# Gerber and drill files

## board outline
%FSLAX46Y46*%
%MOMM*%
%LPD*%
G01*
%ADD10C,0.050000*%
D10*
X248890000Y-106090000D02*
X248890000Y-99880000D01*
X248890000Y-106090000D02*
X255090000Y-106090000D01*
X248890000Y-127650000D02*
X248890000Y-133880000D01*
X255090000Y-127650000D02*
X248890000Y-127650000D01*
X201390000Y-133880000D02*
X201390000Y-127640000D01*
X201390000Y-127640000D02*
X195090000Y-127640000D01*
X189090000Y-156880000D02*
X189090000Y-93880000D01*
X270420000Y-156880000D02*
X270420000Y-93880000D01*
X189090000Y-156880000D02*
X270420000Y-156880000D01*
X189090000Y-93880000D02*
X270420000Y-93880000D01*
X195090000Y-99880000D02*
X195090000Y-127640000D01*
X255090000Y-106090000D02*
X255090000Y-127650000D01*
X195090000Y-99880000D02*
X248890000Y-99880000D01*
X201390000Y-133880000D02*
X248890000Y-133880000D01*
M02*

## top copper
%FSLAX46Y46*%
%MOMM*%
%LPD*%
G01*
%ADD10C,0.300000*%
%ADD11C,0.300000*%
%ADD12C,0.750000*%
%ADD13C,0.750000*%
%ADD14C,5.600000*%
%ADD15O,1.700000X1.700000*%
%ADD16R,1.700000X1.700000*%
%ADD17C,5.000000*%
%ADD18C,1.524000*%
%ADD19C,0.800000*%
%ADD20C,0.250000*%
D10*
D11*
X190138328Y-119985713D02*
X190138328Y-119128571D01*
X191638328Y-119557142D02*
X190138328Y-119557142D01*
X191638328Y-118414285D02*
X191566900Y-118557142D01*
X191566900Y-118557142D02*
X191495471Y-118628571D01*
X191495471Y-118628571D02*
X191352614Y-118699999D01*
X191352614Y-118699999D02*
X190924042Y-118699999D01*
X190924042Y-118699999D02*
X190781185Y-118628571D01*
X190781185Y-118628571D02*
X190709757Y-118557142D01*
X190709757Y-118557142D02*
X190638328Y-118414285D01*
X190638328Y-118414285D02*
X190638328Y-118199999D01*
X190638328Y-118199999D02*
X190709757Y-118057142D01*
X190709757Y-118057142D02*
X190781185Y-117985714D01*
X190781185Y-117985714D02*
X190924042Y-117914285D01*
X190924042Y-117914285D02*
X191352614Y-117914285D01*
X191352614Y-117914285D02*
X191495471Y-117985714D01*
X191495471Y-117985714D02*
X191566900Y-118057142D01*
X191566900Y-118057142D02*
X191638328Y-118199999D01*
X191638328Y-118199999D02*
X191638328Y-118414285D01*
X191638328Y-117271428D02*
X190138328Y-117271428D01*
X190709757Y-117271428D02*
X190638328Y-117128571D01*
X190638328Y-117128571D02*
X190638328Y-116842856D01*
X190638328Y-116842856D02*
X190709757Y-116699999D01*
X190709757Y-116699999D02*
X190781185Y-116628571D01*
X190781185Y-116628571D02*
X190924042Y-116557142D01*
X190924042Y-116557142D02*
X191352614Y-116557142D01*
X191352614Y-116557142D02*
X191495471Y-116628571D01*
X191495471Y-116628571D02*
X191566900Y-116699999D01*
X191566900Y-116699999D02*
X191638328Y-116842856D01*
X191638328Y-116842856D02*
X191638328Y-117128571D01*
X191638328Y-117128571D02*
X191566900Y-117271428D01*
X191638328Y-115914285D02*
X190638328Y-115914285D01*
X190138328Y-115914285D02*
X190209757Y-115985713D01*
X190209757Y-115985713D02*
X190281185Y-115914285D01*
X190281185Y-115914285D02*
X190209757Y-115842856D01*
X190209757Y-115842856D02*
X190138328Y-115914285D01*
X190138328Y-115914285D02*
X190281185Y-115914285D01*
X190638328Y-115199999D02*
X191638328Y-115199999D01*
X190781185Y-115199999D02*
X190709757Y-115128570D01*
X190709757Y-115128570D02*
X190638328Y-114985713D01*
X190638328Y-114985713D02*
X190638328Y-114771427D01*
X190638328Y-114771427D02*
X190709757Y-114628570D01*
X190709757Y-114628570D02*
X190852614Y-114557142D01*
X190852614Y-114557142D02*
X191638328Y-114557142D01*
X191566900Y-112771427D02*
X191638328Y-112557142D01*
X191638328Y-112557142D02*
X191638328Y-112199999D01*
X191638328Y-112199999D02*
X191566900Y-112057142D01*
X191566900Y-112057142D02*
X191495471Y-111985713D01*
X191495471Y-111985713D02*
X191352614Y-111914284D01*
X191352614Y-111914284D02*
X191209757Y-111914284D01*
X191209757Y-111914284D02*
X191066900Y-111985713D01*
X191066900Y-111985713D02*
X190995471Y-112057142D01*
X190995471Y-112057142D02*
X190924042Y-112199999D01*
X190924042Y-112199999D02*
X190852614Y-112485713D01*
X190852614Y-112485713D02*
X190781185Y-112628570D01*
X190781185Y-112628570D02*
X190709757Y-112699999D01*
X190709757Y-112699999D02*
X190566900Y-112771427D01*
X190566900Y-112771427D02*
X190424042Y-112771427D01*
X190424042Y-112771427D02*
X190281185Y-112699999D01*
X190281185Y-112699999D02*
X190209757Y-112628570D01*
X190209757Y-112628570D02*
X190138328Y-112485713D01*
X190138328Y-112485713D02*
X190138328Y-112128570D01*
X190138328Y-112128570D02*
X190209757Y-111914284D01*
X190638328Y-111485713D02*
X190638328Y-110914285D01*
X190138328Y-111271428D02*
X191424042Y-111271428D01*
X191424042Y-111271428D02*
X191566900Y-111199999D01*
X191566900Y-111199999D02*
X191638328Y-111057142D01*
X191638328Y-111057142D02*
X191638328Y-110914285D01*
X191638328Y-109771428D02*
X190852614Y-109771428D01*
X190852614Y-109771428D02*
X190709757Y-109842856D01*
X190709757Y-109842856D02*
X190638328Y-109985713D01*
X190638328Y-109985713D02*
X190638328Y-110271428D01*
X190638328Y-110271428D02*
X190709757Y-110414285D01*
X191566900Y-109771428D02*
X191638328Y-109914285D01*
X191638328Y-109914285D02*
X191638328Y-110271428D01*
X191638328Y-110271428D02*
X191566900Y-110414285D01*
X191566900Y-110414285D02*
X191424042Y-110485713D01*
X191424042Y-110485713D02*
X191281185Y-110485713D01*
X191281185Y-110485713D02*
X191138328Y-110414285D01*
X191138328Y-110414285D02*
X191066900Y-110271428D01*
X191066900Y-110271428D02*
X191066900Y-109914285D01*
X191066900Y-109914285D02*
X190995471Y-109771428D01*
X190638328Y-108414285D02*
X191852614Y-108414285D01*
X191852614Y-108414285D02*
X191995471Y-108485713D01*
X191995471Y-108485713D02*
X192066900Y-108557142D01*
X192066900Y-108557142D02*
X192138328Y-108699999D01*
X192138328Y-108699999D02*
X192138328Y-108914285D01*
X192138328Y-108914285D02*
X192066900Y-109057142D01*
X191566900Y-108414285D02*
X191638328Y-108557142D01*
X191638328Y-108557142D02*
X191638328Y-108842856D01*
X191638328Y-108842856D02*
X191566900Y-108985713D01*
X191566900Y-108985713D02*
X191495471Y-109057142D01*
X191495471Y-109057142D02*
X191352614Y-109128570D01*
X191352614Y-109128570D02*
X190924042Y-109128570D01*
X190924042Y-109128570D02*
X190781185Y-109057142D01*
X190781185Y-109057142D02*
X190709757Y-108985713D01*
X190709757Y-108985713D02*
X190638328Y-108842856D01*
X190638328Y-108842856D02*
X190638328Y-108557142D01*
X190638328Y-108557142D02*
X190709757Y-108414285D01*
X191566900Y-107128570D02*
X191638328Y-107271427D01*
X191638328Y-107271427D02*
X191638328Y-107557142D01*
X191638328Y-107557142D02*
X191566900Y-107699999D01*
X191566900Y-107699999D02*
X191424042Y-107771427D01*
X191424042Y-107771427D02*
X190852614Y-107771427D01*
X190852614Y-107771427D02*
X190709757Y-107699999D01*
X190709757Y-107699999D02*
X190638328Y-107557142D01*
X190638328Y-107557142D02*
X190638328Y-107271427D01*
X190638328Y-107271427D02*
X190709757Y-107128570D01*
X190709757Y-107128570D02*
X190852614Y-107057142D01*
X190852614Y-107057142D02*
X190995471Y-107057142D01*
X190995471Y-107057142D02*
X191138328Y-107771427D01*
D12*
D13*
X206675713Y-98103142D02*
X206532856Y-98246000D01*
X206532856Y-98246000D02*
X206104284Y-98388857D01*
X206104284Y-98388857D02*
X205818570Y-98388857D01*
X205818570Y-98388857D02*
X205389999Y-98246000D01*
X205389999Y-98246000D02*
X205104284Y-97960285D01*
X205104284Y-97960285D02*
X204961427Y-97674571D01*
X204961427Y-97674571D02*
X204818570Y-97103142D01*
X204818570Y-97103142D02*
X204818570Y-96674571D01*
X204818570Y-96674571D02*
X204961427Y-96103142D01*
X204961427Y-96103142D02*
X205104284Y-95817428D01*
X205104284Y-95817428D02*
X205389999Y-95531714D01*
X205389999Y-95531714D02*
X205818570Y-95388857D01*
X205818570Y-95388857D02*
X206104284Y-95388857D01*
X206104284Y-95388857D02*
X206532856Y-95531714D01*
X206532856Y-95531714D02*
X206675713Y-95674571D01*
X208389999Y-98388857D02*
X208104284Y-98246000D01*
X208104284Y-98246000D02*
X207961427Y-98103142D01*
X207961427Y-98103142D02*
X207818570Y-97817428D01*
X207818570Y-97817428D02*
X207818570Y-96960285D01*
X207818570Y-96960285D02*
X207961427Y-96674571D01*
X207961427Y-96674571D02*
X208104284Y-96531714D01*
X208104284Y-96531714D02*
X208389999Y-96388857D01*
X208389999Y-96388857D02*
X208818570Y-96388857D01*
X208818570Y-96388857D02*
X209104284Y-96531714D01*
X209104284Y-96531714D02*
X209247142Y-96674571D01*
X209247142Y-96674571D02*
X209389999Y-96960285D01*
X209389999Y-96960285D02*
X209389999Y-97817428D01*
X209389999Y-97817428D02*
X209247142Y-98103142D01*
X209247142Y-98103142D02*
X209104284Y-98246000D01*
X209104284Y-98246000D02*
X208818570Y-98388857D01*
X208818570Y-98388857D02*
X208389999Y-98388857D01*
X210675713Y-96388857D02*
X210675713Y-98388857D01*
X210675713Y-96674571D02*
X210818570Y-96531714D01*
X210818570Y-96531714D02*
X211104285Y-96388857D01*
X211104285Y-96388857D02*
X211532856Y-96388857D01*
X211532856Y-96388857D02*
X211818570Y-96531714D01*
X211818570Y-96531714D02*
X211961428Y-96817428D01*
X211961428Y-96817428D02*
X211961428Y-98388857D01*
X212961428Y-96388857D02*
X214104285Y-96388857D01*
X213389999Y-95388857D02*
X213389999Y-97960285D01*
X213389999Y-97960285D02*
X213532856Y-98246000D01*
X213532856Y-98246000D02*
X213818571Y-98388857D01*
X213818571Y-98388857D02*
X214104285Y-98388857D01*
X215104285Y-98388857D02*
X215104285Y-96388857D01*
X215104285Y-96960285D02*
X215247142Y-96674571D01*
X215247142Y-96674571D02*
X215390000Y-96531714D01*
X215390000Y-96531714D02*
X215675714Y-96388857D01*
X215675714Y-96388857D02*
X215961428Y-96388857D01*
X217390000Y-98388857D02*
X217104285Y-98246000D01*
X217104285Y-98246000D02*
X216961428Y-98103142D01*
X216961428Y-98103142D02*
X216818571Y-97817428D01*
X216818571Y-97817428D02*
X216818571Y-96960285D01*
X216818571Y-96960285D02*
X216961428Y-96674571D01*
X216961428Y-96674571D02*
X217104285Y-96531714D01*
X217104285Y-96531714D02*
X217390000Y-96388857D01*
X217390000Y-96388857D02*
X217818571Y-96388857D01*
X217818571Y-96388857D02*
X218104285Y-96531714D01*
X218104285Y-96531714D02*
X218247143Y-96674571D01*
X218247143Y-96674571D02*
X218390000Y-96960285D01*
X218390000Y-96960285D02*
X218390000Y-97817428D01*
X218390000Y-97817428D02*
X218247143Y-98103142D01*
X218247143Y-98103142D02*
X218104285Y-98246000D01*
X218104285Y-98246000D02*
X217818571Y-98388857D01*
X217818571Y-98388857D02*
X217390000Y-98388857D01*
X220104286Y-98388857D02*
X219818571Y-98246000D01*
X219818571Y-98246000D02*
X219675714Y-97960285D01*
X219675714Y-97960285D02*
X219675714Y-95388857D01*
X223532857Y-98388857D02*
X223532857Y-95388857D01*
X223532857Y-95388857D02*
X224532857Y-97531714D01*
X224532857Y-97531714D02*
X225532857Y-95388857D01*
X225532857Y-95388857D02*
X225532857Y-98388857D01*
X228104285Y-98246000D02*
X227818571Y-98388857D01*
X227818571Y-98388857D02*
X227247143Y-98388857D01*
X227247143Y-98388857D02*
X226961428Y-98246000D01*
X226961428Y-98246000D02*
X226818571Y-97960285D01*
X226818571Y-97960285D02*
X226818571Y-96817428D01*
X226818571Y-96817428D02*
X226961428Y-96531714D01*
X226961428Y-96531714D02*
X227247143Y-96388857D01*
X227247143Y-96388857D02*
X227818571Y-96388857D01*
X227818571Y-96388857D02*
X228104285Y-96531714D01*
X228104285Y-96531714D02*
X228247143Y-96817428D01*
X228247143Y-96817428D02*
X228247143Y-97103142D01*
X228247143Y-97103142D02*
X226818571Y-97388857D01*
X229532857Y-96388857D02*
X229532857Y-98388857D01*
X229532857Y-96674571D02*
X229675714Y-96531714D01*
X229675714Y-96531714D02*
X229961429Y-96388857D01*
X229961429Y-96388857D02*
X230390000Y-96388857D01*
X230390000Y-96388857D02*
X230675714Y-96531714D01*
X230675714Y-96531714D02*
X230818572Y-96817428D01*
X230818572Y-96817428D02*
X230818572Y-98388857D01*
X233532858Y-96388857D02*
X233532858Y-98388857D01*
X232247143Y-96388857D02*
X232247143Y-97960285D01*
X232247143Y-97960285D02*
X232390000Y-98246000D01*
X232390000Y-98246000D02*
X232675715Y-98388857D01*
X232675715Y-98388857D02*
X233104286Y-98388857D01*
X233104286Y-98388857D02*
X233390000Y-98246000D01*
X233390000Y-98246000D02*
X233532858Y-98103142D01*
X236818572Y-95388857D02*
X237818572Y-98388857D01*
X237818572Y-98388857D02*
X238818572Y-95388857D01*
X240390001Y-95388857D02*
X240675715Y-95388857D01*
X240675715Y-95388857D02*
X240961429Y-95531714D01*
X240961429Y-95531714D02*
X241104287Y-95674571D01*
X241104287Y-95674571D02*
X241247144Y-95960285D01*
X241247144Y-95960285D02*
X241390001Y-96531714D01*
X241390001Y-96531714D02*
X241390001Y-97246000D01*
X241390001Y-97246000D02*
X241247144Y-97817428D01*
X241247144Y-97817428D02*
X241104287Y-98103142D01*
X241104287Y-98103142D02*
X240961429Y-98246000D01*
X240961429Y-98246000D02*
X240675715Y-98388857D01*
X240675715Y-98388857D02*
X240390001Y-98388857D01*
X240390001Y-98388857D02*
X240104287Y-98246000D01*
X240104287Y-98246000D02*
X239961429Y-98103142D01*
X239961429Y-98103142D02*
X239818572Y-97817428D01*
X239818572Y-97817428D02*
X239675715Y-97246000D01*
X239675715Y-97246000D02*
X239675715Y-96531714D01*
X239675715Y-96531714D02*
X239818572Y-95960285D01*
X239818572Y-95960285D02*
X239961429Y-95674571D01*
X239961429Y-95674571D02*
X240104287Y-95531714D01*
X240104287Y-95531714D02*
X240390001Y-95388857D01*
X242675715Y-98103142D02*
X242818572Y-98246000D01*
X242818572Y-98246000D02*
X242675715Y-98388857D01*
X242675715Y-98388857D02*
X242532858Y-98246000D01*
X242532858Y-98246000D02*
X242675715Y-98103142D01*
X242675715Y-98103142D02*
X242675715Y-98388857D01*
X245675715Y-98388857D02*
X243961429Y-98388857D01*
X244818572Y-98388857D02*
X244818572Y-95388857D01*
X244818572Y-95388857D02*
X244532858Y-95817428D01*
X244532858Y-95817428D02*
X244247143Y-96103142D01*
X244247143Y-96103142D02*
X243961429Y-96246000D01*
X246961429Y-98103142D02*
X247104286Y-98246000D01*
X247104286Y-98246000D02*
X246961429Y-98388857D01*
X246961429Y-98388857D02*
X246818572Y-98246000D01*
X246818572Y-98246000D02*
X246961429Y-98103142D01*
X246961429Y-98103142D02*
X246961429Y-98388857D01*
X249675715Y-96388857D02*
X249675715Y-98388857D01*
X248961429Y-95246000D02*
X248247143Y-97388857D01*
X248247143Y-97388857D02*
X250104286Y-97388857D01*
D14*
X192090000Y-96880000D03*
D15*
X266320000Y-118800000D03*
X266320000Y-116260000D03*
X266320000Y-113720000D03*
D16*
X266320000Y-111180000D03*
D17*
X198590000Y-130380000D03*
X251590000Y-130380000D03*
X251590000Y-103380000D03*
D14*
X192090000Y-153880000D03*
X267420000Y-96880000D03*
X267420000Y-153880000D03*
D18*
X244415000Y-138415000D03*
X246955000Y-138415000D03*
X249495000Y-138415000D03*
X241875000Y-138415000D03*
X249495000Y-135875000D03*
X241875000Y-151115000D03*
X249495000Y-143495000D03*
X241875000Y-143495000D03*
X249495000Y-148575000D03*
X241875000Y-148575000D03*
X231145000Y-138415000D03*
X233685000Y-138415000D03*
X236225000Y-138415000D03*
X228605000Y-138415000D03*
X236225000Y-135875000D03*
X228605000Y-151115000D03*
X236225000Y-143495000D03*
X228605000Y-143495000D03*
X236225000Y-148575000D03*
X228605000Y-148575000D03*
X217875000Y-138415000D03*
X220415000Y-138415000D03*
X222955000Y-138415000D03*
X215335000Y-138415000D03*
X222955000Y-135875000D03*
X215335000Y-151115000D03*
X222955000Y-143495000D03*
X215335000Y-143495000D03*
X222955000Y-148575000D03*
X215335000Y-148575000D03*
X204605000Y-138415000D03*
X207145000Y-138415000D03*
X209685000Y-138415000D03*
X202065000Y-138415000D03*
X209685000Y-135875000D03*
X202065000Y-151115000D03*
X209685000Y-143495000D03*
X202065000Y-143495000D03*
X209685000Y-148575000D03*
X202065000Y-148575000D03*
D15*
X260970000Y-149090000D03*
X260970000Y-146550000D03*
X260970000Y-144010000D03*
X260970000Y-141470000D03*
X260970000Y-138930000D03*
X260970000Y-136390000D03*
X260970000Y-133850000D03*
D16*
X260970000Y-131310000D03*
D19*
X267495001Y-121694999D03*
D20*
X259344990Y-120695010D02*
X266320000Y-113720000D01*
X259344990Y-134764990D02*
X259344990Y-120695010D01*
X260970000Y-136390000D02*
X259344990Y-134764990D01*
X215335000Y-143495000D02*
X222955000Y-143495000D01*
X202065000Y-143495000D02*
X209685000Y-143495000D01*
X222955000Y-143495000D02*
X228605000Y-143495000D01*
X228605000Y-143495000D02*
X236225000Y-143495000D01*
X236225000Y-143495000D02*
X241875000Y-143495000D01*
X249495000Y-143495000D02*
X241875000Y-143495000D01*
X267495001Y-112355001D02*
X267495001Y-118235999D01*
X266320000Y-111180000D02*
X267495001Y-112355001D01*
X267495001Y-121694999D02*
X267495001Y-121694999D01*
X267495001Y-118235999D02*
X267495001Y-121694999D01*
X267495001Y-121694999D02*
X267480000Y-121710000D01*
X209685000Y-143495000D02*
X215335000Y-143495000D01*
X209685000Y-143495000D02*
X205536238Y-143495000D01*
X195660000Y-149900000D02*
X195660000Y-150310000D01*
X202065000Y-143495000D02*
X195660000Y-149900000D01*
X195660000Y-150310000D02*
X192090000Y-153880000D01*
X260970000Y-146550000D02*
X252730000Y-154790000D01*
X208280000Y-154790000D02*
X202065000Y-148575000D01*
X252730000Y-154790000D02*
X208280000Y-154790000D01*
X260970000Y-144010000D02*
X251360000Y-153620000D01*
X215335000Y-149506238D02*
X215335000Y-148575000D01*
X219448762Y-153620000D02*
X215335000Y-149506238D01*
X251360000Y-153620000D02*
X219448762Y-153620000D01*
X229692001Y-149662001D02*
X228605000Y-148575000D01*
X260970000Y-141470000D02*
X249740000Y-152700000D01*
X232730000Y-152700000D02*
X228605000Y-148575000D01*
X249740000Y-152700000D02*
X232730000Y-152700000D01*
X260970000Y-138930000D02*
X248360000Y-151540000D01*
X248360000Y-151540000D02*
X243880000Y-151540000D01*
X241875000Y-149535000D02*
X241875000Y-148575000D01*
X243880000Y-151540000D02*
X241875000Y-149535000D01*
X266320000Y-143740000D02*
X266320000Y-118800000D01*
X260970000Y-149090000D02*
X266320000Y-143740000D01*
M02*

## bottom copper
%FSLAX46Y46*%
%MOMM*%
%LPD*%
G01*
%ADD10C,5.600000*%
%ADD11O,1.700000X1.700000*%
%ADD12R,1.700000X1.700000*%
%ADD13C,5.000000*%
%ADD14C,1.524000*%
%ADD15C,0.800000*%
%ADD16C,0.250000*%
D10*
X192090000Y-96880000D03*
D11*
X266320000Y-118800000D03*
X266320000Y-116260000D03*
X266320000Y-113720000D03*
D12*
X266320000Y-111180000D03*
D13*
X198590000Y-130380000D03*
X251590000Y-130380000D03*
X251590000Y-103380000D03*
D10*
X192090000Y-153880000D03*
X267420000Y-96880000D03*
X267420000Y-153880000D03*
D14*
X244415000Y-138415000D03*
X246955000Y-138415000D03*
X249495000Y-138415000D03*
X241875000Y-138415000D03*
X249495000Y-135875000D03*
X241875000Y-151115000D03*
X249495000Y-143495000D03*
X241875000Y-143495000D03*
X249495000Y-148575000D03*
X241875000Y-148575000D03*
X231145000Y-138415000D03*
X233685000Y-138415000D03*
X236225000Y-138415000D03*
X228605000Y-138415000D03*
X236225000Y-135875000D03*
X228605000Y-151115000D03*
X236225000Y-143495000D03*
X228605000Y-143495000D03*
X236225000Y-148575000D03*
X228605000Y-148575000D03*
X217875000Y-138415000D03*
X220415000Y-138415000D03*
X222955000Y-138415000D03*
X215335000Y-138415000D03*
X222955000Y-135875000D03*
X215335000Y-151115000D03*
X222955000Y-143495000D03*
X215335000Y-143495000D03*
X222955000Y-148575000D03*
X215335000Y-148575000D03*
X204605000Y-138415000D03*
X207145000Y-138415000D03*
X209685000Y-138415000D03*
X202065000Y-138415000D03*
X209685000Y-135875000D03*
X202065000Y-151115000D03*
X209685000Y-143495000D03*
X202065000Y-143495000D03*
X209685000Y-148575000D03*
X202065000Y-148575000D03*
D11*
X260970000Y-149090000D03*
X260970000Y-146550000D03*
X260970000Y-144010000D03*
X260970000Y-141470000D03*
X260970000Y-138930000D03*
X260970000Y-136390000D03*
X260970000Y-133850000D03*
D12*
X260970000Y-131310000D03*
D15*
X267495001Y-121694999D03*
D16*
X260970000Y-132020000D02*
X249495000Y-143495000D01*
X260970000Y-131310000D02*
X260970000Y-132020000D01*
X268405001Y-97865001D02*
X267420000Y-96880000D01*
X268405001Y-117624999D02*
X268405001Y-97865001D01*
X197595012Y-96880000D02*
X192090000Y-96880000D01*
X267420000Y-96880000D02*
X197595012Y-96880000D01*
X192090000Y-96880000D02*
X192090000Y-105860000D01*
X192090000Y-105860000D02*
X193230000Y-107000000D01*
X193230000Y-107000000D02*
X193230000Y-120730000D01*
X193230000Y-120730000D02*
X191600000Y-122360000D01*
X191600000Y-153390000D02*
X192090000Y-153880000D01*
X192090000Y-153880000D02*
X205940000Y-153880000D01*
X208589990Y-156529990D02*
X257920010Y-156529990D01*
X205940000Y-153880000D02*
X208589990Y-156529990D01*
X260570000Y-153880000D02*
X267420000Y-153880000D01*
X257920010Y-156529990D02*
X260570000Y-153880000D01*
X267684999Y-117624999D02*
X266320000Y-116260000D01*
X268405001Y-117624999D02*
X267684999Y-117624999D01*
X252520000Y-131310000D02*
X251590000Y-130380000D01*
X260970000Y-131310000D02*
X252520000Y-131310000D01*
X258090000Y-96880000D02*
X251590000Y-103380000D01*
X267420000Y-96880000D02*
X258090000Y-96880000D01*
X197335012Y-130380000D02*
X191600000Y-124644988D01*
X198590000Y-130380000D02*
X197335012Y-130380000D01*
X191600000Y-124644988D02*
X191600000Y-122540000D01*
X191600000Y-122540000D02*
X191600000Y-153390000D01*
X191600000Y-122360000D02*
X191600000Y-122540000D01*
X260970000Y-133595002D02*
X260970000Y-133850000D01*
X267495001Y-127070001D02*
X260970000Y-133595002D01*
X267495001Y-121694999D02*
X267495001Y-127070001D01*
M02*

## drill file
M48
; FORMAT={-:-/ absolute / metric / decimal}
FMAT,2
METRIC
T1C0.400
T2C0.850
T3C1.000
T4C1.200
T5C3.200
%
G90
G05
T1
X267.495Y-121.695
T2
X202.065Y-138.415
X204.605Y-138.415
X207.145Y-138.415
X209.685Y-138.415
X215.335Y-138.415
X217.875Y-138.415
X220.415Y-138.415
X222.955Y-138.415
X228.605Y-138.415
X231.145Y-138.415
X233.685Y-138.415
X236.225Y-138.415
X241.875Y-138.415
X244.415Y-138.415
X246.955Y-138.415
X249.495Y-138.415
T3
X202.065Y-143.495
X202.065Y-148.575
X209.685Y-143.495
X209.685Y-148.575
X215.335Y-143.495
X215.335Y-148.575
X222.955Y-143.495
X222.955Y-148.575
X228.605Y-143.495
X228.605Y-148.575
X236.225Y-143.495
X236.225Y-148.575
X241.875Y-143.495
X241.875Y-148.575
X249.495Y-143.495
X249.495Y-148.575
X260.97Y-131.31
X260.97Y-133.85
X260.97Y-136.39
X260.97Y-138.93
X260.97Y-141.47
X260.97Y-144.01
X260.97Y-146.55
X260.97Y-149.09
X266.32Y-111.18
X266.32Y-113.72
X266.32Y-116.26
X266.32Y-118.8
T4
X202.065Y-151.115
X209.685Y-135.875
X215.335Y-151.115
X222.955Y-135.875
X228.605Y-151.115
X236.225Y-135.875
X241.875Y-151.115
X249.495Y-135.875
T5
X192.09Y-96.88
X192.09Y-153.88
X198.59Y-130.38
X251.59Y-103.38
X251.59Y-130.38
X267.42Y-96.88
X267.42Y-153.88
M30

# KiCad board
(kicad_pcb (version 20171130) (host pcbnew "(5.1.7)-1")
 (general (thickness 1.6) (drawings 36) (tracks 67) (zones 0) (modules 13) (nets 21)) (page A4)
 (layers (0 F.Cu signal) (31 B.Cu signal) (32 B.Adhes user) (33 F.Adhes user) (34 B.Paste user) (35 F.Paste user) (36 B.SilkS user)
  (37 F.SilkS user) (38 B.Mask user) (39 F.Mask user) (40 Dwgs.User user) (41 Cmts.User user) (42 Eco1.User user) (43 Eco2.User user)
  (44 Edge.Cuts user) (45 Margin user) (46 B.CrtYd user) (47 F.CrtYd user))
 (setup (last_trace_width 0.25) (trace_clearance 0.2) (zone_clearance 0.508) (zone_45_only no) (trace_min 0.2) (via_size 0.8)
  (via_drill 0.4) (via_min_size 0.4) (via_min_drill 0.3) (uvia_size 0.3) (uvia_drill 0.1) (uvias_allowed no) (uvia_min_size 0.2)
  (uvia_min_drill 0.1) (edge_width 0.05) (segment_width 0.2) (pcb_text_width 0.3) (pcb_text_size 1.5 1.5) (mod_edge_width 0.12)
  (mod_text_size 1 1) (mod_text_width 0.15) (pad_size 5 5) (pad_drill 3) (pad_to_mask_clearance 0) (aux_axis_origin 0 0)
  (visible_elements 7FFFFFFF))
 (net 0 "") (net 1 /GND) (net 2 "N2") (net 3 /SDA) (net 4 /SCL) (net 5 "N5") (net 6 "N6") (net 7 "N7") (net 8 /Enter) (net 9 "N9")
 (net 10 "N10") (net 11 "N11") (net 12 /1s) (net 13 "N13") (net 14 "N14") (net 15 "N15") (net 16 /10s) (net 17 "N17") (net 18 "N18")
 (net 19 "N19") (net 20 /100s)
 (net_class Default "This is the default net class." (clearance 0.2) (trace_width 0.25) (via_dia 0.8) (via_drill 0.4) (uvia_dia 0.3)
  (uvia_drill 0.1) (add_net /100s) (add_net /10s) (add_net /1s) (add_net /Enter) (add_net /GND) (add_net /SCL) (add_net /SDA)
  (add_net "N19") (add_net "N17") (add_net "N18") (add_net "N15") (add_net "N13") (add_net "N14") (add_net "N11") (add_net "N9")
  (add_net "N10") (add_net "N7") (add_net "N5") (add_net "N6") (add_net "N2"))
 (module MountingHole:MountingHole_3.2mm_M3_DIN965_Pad (layer F.Cu) (at 192.09 96.88)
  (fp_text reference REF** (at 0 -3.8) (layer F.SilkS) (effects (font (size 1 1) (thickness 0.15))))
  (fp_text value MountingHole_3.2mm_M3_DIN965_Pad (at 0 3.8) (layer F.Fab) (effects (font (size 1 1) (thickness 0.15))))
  (pad 1 thru_hole circle (at 0 0) (size 5.6 5.6) (drill 3.2) (layers *.Cu *.Mask) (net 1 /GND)))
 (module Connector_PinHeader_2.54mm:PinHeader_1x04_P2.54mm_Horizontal (layer B.Cu) (at 266.32 111.18 180)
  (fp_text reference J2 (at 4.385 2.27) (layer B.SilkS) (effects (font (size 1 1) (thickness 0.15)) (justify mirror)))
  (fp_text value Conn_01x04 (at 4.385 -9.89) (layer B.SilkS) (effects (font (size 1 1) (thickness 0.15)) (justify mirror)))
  (pad 4 thru_hole oval (at 0 -7.62 180) (size 1.7 1.7) (drill 1) (layers *.Cu *.Mask) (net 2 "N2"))
  (pad 3 thru_hole oval (at 0 -5.08 180) (size 1.7 1.7) (drill 1) (layers *.Cu *.Mask) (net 1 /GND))
  (pad 2 thru_hole oval (at 0 -2.54 180) (size 1.7 1.7) (drill 1) (layers *.Cu *.Mask) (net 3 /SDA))
  (pad 1 thru_hole rect (at 0 0 180) (size 1.7 1.7) (drill 1) (layers *.Cu *.Mask) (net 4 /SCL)))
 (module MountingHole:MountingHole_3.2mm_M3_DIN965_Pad (layer F.Cu) (at 198.59 130.38)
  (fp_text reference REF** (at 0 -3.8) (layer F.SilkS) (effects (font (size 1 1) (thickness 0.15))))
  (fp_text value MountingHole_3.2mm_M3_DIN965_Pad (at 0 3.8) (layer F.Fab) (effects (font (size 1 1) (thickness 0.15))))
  (pad 1 thru_hole circle (at 0 0) (size 5 5) (drill 3.2) (layers *.Cu *.Mask) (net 1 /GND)))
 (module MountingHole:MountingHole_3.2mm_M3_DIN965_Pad (layer F.Cu) (at 251.59 130.38)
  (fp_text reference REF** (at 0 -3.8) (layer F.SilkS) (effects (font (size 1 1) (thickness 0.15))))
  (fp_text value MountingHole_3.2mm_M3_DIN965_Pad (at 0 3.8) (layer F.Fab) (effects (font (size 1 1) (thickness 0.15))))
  (pad 1 thru_hole circle (at 0 0) (size 5 5) (drill 3.2) (layers *.Cu *.Mask) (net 1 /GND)))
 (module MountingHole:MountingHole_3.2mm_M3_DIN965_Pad (layer F.Cu) (at 251.59 103.38)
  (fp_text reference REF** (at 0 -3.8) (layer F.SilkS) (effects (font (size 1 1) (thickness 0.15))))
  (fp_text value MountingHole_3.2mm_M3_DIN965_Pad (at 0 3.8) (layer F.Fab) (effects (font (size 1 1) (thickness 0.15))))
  (pad 1 thru_hole circle (at 0 0) (size 5 5) (drill 3.2) (layers *.Cu *.Mask) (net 1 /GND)))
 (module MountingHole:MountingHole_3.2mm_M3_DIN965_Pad (layer F.Cu) (at 192.09 153.88)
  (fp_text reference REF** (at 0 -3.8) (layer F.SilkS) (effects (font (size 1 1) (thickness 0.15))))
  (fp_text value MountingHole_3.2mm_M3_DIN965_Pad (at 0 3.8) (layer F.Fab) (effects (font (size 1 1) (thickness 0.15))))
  (pad 1 thru_hole circle (at 0 0) (size 5.6 5.6) (drill 3.2) (layers *.Cu *.Mask) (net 1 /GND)))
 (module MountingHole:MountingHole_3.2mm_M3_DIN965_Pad (layer F.Cu) (at 267.42 96.88)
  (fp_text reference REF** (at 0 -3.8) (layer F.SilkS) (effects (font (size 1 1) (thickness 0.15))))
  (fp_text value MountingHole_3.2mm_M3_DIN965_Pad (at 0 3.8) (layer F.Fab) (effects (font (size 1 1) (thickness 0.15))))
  (pad 1 thru_hole circle (at 0 0) (size 5.6 5.6) (drill 3.2) (layers *.Cu *.Mask) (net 1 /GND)))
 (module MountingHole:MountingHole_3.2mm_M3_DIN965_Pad (layer F.Cu) (at 267.42 153.88)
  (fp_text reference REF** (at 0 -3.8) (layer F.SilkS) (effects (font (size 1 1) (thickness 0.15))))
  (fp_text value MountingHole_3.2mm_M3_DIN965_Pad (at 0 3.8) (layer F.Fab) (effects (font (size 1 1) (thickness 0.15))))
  (pad 1 thru_hole circle (at 0 0) (size 5.6 5.6) (drill 3.2) (layers *.Cu *.Mask) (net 1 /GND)))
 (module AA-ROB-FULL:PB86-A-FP (layer F.Cu) (at 239.515 134.995)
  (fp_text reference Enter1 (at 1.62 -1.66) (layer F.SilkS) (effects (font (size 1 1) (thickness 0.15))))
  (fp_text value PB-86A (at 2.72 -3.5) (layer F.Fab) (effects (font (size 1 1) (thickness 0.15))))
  (pad 5 thru_hole circle (at 4.9 3.42) (size 1.524 1.524) (drill 0.85) (layers *.Cu *.Mask) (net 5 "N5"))
  (pad 6 thru_hole circle (at 7.44 3.42) (size 1.524 1.524) (drill 0.85) (layers *.Cu *.Mask) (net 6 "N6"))
  (pad 7 thru_hole circle (at 9.98 3.42) (size 1.524 1.524) (drill 0.85) (layers *.Cu *.Mask))
  (pad 4 thru_hole circle (at 2.36 3.42) (size 1.524 1.524) (drill 0.85) (layers *.Cu *.Mask))
  (pad 8 thru_hole circle (at 9.98 0.88) (size 1.524 1.524) (drill 1.2) (layers *.Cu *.Mask))
  (pad 8 thru_hole circle (at 2.36 16.12) (size 1.524 1.524) (drill 1.2) (layers *.Cu *.Mask))
  (pad 1 thru_hole circle (at 9.98 8.5) (size 1.524 1.524) (drill 1) (layers *.Cu *.Mask) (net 1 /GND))
  (pad 1 thru_hole circle (at 2.36 8.5) (size 1.524 1.524) (drill 1) (layers *.Cu *.Mask) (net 1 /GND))
  (pad 3 thru_hole circle (at 9.98 13.58) (size 1.524 1.524) (drill 1) (layers *.Cu *.Mask) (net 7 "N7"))
  (pad 2 thru_hole circle (at 2.36 13.58) (size 1.524 1.524) (drill 1) (layers *.Cu *.Mask) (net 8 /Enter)))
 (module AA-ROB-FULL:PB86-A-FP (layer F.Cu) (at 226.245 134.995)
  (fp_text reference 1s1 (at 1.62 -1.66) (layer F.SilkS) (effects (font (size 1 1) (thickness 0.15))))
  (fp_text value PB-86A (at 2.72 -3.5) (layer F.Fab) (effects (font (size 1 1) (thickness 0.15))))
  (pad 5 thru_hole circle (at 4.9 3.42) (size 1.524 1.524) (drill 0.85) (layers *.Cu *.Mask) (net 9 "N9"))
  (pad 6 thru_hole circle (at 7.44 3.42) (size 1.524 1.524) (drill 0.85) (layers *.Cu *.Mask) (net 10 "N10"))
  (pad 7 thru_hole circle (at 9.98 3.42) (size 1.524 1.524) (drill 0.85) (layers *.Cu *.Mask))
  (pad 4 thru_hole circle (at 2.36 3.42) (size 1.524 1.524) (drill 0.85) (layers *.Cu *.Mask))
  (pad 8 thru_hole circle (at 9.98 0.88) (size 1.524 1.524) (drill 1.2) (layers *.Cu *.Mask))
  (pad 8 thru_hole circle (at 2.36 16.12) (size 1.524 1.524) (drill 1.2) (layers *.Cu *.Mask))
  (pad 1 thru_hole circle (at 9.98 8.5) (size 1.524 1.524) (drill 1) (layers *.Cu *.Mask) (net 1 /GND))
  (pad 1 thru_hole circle (at 2.36 8.5) (size 1.524 1.524) (drill 1) (layers *.Cu *.Mask) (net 1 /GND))
  (pad 3 thru_hole circle (at 9.98 13.58) (size 1.524 1.524) (drill 1) (layers *.Cu *.Mask) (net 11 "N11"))
  (pad 2 thru_hole circle (at 2.36 13.58) (size 1.524 1.524) (drill 1) (layers *.Cu *.Mask) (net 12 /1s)))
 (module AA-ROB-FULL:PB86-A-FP (layer F.Cu) (at 212.975 134.995)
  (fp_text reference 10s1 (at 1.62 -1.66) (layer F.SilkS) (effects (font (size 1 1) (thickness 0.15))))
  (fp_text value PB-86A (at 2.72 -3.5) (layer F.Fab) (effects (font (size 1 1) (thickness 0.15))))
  (pad 5 thru_hole circle (at 4.9 3.42) (size 1.524 1.524) (drill 0.85) (layers *.Cu *.Mask) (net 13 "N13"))
  (pad 6 thru_hole circle (at 7.44 3.42) (size 1.524 1.524) (drill 0.85) (layers *.Cu *.Mask) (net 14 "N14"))
  (pad 7 thru_hole circle (at 9.98 3.42) (size 1.524 1.524) (drill 0.85) (layers *.Cu *.Mask))
  (pad 4 thru_hole circle (at 2.36 3.42) (size 1.524 1.524) (drill 0.85) (layers *.Cu *.Mask))
  (pad 8 thru_hole circle (at 9.98 0.88) (size 1.524 1.524) (drill 1.2) (layers *.Cu *.Mask))
  (pad 8 thru_hole circle (at 2.36 16.12) (size 1.524 1.524) (drill 1.2) (layers *.Cu *.Mask))
  (pad 1 thru_hole circle (at 9.98 8.5) (size 1.524 1.524) (drill 1) (layers *.Cu *.Mask) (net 1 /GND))
  (pad 1 thru_hole circle (at 2.36 8.5) (size 1.524 1.524) (drill 1) (layers *.Cu *.Mask) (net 1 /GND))
  (pad 3 thru_hole circle (at 9.98 13.58) (size 1.524 1.524) (drill 1) (layers *.Cu *.Mask) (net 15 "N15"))
  (pad 2 thru_hole circle (at 2.36 13.58) (size 1.524 1.524) (drill 1) (layers *.Cu *.Mask) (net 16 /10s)))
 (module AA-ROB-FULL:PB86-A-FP (layer F.Cu) (at 199.705 134.995)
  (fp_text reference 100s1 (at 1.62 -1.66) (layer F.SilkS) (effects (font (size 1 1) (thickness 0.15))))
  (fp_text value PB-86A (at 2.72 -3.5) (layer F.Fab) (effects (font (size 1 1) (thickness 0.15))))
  (pad 5 thru_hole circle (at 4.9 3.42) (size 1.524 1.524) (drill 0.85) (layers *.Cu *.Mask) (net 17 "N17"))
  (pad 6 thru_hole circle (at 7.44 3.42) (size 1.524 1.524) (drill 0.85) (layers *.Cu *.Mask) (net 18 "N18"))
  (pad 7 thru_hole circle (at 9.98 3.42) (size 1.524 1.524) (drill 0.85) (layers *.Cu *.Mask))
  (pad 4 thru_hole circle (at 2.36 3.42) (size 1.524 1.524) (drill 0.85) (layers *.Cu *.Mask))
  (pad 8 thru_hole circle (at 9.98 0.88) (size 1.524 1.524) (drill 1.2) (layers *.Cu *.Mask))
  (pad 8 thru_hole circle (at 2.36 16.12) (size 1.524 1.524) (drill 1.2) (layers *.Cu *.Mask))
  (pad 1 thru_hole circle (at 9.98 8.5) (size 1.524 1.524) (drill 1) (layers *.Cu *.Mask) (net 1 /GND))
  (pad 1 thru_hole circle (at 2.36 8.5) (size 1.524 1.524) (drill 1) (layers *.Cu *.Mask) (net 1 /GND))
  (pad 3 thru_hole circle (at 9.98 13.58) (size 1.524 1.524) (drill 1) (layers *.Cu *.Mask) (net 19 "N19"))
  (pad 2 thru_hole circle (at 2.36 13.58) (size 1.524 1.524) (drill 1) (layers *.Cu *.Mask) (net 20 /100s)))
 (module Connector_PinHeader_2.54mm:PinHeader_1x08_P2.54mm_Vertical (layer F.Cu) (at 260.97 131.31)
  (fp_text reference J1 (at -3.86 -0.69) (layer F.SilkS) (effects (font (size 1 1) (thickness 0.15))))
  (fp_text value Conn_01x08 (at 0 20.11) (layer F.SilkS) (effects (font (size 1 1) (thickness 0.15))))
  (pad 8 thru_hole oval (at 0 17.78) (size 1.7 1.7) (drill 1) (layers *.Cu *.Mask) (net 2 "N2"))
  (pad 7 thru_hole oval (at 0 15.24) (size 1.7 1.7) (drill 1) (layers *.Cu *.Mask) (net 20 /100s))
  (pad 6 thru_hole oval (at 0 12.7) (size 1.7 1.7) (drill 1) (layers *.Cu *.Mask) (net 16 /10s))
  (pad 5 thru_hole oval (at 0 10.16) (size 1.7 1.7) (drill 1) (layers *.Cu *.Mask) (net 12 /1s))
  (pad 4 thru_hole oval (at 0 7.62) (size 1.7 1.7) (drill 1) (layers *.Cu *.Mask) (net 8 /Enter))
  (pad 3 thru_hole oval (at 0 5.08) (size 1.7 1.7) (drill 1) (layers *.Cu *.Mask) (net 3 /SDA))
  (pad 2 thru_hole oval (at 0 2.54) (size 1.7 1.7) (drill 1) (layers *.Cu *.Mask) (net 4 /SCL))
  (pad 1 thru_hole rect (at 0 0) (size 1.7 1.7) (drill 1) (layers *.Cu *.Mask) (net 1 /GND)))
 (gr_line (start 248.89 106.09) (end 248.89 99.88) (layer Edge.Cuts) (width 0.05))
 (gr_line (start 248.89 106.09) (end 255.09 106.09) (layer Edge.Cuts) (width 0.05))
 (gr_line (start 248.89 127.65) (end 248.89 133.88) (layer Edge.Cuts) (width 0.05))
 (gr_line (start 255.09 127.65) (end 248.89 127.65) (layer Edge.Cuts) (width 0.05))
 (gr_line (start 201.39 133.88) (end 201.39 127.64) (layer Edge.Cuts) (width 0.05))
 (gr_line (start 201.39 127.64) (end 195.09 127.64) (layer Edge.Cuts) (width 0.05))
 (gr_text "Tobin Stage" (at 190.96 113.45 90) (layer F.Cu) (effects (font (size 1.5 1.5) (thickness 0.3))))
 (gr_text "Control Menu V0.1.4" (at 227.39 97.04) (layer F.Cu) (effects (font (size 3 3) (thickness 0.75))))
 (gr_line (start 189.09 156.88) (end 189.09 93.88) (layer Edge.Cuts) (width 0.05))
 (gr_line (start 270.42 156.88) (end 270.42 93.88) (layer Edge.Cuts) (width 0.05))
 (gr_line (start 189.09 156.88) (end 270.42 156.88) (layer Edge.Cuts) (width 0.05))
 (gr_line (start 189.09 93.88) (end 270.42 93.88) (layer Edge.Cuts) (width 0.05))
 (gr_line (start 195.09 99.88) (end 195.09 127.64) (layer Edge.Cuts) (width 0.05))
 (gr_line (start 255.09 106.09) (end 255.09 127.65) (layer Edge.Cuts) (width 0.05))
 (gr_line (start 195.09 99.88) (end 248.89 99.88) (layer Edge.Cuts) (width 0.05))
 (gr_line (start 201.39 133.88) (end 248.89 133.88) (layer Edge.Cuts) (width 0.05))
 (segment (start 259.34499 120.69501) (end 266.32 113.72) (width 0.25) (layer F.Cu) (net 3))
 (segment (start 259.34499 134.76499) (end 259.34499 120.69501) (width 0.25) (layer F.Cu) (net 3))
 (segment (start 260.97 136.39) (end 259.34499 134.76499) (width 0.25) (layer F.Cu) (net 3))
 (segment (start 215.335 143.495) (end 222.955 143.495) (width 0.25) (layer F.Cu) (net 1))
 (segment (start 202.065 143.495) (end 209.685 143.495) (width 0.25) (layer F.Cu) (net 1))
 (segment (start 222.955 143.495) (end 228.605 143.495) (width 0.25) (layer F.Cu) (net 1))
 (segment (start 228.605 143.495) (end 236.225 143.495) (width 0.25) (layer F.Cu) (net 1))
 (segment (start 236.225 143.495) (end 241.875 143.495) (width 0.25) (layer F.Cu) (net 1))
 (segment (start 249.495 143.495) (end 241.875 143.495) (width 0.25) (layer F.Cu) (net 1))
 (segment (start 260.97 132.02) (end 249.495 143.495) (width 0.25) (layer B.Cu) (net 1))
 (segment (start 260.97 131.31) (end 260.97 132.02) (width 0.25) (layer B.Cu) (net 1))
 (segment (start 268.405001 97.865001) (end 267.42 96.88) (width 0.25) (layer B.Cu) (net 1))
 (segment (start 268.405001 117.624999) (end 268.405001 97.865001) (width 0.25) (layer B.Cu) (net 1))
 (segment (start 197.595012 96.88) (end 192.09 96.88) (width 0.25) (layer B.Cu) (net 1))
 (segment (start 267.42 96.88) (end 197.595012 96.88) (width 0.25) (layer B.Cu) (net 1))
 (segment (start 192.09 96.88) (end 192.09 105.86) (width 0.25) (layer B.Cu) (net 1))
 (segment (start 192.09 105.86) (end 193.23 107) (width 0.25) (layer B.Cu) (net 1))
 (segment (start 193.23 107) (end 193.23 120.73) (width 0.25) (layer B.Cu) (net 1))
 (segment (start 193.23 120.73) (end 191.6 122.36) (width 0.25) (layer B.Cu) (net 1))
 (segment (start 191.6 153.39) (end 192.09 153.88) (width 0.25) (layer B.Cu) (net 1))
 (segment (start 192.09 153.88) (end 205.94 153.88) (width 0.25) (layer B.Cu) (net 1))
 (segment (start 208.58999 156.52999) (end 257.92001 156.52999) (width 0.25) (layer B.Cu) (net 1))
 (segment (start 205.94 153.88) (end 208.58999 156.52999) (width 0.25) (layer B.Cu) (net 1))
 (segment (start 260.57 153.88) (end 267.42 153.88) (width 0.25) (layer B.Cu) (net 1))
 (segment (start 257.92001 156.52999) (end 260.57 153.88) (width 0.25) (layer B.Cu) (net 1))
 (segment (start 267.684999 117.624999) (end 266.32 116.26) (width 0.25) (layer B.Cu) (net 1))
 (segment (start 268.405001 117.624999) (end 267.684999 117.624999) (width 0.25) (layer B.Cu) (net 1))
 (segment (start 252.52 131.31) (end 251.59 130.38) (width 0.25) (layer B.Cu) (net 1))
 (segment (start 260.97 131.31) (end 252.52 131.31) (width 0.25) (layer B.Cu) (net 1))
 (segment (start 258.09 96.88) (end 251.59 103.38) (width 0.25) (layer B.Cu) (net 1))
 (segment (start 267.42 96.88) (end 258.09 96.88) (width 0.25) (layer B.Cu) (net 1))
 (segment (start 197.335012 130.38) (end 191.6 124.644988) (width 0.25) (layer B.Cu) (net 1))
 (segment (start 198.59 130.38) (end 197.335012 130.38) (width 0.25) (layer B.Cu) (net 1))
 (segment (start 191.6 124.644988) (end 191.6 122.54) (width 0.25) (layer B.Cu) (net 1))
 (segment (start 191.6 122.54) (end 191.6 153.39) (width 0.25) (layer B.Cu) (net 1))
 (segment (start 191.6 122.36) (end 191.6 122.54) (width 0.25) (layer B.Cu) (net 1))
 (segment (start 267.495001 112.355001) (end 267.495001 118.235999) (width 0.25) (layer F.Cu) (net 4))
 (segment (start 266.32 111.18) (end 267.495001 112.355001) (width 0.25) (layer F.Cu) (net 4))
 (segment (start 267.495001 121.694999) (end 267.495001 121.694999) (width 0.25) (layer F.Cu) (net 4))
 (segment (start 267.495001 118.235999) (end 267.495001 121.694999) (width 0.25) (layer F.Cu) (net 4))
 (segment (start 267.495001 121.694999) (end 267.48 121.71) (width 0.25) (layer F.Cu) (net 4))
 (via (at 267.495001 121.694999) (size 0.8) (drill 0.4) (layers F.Cu B.Cu) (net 4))
 (segment (start 260.97 133.595002) (end 260.97 133.85) (width 0.25) (layer B.Cu) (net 4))
 (segment (start 267.495001 127.070001) (end 260.97 133.595002) (width 0.25) (layer B.Cu) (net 4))
 (segment (start 267.495001 121.694999) (end 267.495001 127.070001) (width 0.25) (layer B.Cu) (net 4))
 (segment (start 209.685 143.495) (end 215.335 143.495) (width 0.25) (layer F.Cu) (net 1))
 (segment (start 209.685 143.495) (end 205.536238 143.495) (width 0.25) (layer F.Cu) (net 1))
 (segment (start 195.66 149.9) (end 195.66 150.31) (width 0.25) (layer F.Cu) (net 1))
 (segment (start 202.065 143.495) (end 195.66 149.9) (width 0.25) (layer F.Cu) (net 1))
 (segment (start 195.66 150.31) (end 192.09 153.88) (width 0.25) (layer F.Cu) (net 1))
 (segment (start 260.97 146.55) (end 252.73 154.79) (width 0.25) (layer F.Cu) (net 20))
 (segment (start 208.28 154.79) (end 202.065 148.575) (width 0.25) (layer F.Cu) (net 20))
 (segment (start 252.73 154.79) (end 208.28 154.79) (width 0.25) (layer F.Cu) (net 20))
 (segment (start 260.97 144.01) (end 251.36 153.62) (width 0.25) (layer F.Cu) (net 16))
 (segment (start 215.335 149.506238) (end 215.335 148.575) (width 0.25) (layer F.Cu) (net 16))
 (segment (start 219.448762 153.62) (end 215.335 149.506238) (width 0.25) (layer F.Cu) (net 16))
 (segment (start 251.36 153.62) (end 219.448762 153.62) (width 0.25) (layer F.Cu) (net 16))
 (segment (start 229.692001 149.662001) (end 228.605 148.575) (width 0.25) (layer F.Cu) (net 12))
 (segment (start 260.97 141.47) (end 249.74 152.7) (width 0.25) (layer F.Cu) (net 12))
 (segment (start 232.73 152.7) (end 228.605 148.575) (width 0.25) (layer F.Cu) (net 12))
 (segment (start 249.74 152.7) (end 232.73 152.7) (width 0.25) (layer F.Cu) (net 12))
 (segment (start 260.97 138.93) (end 248.36 151.54) (width 0.25) (layer F.Cu) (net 8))
 (segment (start 248.36 151.54) (end 243.88 151.54) (width 0.25) (layer F.Cu) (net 8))
 (segment (start 241.875 149.535) (end 241.875 148.575) (width 0.25) (layer F.Cu) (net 8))
 (segment (start 243.88 151.54) (end 241.875 149.535) (width 0.25) (layer F.Cu) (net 8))
 (segment (start 266.32 143.74) (end 266.32 118.8) (width 0.25) (layer F.Cu) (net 2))
 (segment (start 260.97 149.09) (end 266.32 143.74) (width 0.25) (layer F.Cu) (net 2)))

